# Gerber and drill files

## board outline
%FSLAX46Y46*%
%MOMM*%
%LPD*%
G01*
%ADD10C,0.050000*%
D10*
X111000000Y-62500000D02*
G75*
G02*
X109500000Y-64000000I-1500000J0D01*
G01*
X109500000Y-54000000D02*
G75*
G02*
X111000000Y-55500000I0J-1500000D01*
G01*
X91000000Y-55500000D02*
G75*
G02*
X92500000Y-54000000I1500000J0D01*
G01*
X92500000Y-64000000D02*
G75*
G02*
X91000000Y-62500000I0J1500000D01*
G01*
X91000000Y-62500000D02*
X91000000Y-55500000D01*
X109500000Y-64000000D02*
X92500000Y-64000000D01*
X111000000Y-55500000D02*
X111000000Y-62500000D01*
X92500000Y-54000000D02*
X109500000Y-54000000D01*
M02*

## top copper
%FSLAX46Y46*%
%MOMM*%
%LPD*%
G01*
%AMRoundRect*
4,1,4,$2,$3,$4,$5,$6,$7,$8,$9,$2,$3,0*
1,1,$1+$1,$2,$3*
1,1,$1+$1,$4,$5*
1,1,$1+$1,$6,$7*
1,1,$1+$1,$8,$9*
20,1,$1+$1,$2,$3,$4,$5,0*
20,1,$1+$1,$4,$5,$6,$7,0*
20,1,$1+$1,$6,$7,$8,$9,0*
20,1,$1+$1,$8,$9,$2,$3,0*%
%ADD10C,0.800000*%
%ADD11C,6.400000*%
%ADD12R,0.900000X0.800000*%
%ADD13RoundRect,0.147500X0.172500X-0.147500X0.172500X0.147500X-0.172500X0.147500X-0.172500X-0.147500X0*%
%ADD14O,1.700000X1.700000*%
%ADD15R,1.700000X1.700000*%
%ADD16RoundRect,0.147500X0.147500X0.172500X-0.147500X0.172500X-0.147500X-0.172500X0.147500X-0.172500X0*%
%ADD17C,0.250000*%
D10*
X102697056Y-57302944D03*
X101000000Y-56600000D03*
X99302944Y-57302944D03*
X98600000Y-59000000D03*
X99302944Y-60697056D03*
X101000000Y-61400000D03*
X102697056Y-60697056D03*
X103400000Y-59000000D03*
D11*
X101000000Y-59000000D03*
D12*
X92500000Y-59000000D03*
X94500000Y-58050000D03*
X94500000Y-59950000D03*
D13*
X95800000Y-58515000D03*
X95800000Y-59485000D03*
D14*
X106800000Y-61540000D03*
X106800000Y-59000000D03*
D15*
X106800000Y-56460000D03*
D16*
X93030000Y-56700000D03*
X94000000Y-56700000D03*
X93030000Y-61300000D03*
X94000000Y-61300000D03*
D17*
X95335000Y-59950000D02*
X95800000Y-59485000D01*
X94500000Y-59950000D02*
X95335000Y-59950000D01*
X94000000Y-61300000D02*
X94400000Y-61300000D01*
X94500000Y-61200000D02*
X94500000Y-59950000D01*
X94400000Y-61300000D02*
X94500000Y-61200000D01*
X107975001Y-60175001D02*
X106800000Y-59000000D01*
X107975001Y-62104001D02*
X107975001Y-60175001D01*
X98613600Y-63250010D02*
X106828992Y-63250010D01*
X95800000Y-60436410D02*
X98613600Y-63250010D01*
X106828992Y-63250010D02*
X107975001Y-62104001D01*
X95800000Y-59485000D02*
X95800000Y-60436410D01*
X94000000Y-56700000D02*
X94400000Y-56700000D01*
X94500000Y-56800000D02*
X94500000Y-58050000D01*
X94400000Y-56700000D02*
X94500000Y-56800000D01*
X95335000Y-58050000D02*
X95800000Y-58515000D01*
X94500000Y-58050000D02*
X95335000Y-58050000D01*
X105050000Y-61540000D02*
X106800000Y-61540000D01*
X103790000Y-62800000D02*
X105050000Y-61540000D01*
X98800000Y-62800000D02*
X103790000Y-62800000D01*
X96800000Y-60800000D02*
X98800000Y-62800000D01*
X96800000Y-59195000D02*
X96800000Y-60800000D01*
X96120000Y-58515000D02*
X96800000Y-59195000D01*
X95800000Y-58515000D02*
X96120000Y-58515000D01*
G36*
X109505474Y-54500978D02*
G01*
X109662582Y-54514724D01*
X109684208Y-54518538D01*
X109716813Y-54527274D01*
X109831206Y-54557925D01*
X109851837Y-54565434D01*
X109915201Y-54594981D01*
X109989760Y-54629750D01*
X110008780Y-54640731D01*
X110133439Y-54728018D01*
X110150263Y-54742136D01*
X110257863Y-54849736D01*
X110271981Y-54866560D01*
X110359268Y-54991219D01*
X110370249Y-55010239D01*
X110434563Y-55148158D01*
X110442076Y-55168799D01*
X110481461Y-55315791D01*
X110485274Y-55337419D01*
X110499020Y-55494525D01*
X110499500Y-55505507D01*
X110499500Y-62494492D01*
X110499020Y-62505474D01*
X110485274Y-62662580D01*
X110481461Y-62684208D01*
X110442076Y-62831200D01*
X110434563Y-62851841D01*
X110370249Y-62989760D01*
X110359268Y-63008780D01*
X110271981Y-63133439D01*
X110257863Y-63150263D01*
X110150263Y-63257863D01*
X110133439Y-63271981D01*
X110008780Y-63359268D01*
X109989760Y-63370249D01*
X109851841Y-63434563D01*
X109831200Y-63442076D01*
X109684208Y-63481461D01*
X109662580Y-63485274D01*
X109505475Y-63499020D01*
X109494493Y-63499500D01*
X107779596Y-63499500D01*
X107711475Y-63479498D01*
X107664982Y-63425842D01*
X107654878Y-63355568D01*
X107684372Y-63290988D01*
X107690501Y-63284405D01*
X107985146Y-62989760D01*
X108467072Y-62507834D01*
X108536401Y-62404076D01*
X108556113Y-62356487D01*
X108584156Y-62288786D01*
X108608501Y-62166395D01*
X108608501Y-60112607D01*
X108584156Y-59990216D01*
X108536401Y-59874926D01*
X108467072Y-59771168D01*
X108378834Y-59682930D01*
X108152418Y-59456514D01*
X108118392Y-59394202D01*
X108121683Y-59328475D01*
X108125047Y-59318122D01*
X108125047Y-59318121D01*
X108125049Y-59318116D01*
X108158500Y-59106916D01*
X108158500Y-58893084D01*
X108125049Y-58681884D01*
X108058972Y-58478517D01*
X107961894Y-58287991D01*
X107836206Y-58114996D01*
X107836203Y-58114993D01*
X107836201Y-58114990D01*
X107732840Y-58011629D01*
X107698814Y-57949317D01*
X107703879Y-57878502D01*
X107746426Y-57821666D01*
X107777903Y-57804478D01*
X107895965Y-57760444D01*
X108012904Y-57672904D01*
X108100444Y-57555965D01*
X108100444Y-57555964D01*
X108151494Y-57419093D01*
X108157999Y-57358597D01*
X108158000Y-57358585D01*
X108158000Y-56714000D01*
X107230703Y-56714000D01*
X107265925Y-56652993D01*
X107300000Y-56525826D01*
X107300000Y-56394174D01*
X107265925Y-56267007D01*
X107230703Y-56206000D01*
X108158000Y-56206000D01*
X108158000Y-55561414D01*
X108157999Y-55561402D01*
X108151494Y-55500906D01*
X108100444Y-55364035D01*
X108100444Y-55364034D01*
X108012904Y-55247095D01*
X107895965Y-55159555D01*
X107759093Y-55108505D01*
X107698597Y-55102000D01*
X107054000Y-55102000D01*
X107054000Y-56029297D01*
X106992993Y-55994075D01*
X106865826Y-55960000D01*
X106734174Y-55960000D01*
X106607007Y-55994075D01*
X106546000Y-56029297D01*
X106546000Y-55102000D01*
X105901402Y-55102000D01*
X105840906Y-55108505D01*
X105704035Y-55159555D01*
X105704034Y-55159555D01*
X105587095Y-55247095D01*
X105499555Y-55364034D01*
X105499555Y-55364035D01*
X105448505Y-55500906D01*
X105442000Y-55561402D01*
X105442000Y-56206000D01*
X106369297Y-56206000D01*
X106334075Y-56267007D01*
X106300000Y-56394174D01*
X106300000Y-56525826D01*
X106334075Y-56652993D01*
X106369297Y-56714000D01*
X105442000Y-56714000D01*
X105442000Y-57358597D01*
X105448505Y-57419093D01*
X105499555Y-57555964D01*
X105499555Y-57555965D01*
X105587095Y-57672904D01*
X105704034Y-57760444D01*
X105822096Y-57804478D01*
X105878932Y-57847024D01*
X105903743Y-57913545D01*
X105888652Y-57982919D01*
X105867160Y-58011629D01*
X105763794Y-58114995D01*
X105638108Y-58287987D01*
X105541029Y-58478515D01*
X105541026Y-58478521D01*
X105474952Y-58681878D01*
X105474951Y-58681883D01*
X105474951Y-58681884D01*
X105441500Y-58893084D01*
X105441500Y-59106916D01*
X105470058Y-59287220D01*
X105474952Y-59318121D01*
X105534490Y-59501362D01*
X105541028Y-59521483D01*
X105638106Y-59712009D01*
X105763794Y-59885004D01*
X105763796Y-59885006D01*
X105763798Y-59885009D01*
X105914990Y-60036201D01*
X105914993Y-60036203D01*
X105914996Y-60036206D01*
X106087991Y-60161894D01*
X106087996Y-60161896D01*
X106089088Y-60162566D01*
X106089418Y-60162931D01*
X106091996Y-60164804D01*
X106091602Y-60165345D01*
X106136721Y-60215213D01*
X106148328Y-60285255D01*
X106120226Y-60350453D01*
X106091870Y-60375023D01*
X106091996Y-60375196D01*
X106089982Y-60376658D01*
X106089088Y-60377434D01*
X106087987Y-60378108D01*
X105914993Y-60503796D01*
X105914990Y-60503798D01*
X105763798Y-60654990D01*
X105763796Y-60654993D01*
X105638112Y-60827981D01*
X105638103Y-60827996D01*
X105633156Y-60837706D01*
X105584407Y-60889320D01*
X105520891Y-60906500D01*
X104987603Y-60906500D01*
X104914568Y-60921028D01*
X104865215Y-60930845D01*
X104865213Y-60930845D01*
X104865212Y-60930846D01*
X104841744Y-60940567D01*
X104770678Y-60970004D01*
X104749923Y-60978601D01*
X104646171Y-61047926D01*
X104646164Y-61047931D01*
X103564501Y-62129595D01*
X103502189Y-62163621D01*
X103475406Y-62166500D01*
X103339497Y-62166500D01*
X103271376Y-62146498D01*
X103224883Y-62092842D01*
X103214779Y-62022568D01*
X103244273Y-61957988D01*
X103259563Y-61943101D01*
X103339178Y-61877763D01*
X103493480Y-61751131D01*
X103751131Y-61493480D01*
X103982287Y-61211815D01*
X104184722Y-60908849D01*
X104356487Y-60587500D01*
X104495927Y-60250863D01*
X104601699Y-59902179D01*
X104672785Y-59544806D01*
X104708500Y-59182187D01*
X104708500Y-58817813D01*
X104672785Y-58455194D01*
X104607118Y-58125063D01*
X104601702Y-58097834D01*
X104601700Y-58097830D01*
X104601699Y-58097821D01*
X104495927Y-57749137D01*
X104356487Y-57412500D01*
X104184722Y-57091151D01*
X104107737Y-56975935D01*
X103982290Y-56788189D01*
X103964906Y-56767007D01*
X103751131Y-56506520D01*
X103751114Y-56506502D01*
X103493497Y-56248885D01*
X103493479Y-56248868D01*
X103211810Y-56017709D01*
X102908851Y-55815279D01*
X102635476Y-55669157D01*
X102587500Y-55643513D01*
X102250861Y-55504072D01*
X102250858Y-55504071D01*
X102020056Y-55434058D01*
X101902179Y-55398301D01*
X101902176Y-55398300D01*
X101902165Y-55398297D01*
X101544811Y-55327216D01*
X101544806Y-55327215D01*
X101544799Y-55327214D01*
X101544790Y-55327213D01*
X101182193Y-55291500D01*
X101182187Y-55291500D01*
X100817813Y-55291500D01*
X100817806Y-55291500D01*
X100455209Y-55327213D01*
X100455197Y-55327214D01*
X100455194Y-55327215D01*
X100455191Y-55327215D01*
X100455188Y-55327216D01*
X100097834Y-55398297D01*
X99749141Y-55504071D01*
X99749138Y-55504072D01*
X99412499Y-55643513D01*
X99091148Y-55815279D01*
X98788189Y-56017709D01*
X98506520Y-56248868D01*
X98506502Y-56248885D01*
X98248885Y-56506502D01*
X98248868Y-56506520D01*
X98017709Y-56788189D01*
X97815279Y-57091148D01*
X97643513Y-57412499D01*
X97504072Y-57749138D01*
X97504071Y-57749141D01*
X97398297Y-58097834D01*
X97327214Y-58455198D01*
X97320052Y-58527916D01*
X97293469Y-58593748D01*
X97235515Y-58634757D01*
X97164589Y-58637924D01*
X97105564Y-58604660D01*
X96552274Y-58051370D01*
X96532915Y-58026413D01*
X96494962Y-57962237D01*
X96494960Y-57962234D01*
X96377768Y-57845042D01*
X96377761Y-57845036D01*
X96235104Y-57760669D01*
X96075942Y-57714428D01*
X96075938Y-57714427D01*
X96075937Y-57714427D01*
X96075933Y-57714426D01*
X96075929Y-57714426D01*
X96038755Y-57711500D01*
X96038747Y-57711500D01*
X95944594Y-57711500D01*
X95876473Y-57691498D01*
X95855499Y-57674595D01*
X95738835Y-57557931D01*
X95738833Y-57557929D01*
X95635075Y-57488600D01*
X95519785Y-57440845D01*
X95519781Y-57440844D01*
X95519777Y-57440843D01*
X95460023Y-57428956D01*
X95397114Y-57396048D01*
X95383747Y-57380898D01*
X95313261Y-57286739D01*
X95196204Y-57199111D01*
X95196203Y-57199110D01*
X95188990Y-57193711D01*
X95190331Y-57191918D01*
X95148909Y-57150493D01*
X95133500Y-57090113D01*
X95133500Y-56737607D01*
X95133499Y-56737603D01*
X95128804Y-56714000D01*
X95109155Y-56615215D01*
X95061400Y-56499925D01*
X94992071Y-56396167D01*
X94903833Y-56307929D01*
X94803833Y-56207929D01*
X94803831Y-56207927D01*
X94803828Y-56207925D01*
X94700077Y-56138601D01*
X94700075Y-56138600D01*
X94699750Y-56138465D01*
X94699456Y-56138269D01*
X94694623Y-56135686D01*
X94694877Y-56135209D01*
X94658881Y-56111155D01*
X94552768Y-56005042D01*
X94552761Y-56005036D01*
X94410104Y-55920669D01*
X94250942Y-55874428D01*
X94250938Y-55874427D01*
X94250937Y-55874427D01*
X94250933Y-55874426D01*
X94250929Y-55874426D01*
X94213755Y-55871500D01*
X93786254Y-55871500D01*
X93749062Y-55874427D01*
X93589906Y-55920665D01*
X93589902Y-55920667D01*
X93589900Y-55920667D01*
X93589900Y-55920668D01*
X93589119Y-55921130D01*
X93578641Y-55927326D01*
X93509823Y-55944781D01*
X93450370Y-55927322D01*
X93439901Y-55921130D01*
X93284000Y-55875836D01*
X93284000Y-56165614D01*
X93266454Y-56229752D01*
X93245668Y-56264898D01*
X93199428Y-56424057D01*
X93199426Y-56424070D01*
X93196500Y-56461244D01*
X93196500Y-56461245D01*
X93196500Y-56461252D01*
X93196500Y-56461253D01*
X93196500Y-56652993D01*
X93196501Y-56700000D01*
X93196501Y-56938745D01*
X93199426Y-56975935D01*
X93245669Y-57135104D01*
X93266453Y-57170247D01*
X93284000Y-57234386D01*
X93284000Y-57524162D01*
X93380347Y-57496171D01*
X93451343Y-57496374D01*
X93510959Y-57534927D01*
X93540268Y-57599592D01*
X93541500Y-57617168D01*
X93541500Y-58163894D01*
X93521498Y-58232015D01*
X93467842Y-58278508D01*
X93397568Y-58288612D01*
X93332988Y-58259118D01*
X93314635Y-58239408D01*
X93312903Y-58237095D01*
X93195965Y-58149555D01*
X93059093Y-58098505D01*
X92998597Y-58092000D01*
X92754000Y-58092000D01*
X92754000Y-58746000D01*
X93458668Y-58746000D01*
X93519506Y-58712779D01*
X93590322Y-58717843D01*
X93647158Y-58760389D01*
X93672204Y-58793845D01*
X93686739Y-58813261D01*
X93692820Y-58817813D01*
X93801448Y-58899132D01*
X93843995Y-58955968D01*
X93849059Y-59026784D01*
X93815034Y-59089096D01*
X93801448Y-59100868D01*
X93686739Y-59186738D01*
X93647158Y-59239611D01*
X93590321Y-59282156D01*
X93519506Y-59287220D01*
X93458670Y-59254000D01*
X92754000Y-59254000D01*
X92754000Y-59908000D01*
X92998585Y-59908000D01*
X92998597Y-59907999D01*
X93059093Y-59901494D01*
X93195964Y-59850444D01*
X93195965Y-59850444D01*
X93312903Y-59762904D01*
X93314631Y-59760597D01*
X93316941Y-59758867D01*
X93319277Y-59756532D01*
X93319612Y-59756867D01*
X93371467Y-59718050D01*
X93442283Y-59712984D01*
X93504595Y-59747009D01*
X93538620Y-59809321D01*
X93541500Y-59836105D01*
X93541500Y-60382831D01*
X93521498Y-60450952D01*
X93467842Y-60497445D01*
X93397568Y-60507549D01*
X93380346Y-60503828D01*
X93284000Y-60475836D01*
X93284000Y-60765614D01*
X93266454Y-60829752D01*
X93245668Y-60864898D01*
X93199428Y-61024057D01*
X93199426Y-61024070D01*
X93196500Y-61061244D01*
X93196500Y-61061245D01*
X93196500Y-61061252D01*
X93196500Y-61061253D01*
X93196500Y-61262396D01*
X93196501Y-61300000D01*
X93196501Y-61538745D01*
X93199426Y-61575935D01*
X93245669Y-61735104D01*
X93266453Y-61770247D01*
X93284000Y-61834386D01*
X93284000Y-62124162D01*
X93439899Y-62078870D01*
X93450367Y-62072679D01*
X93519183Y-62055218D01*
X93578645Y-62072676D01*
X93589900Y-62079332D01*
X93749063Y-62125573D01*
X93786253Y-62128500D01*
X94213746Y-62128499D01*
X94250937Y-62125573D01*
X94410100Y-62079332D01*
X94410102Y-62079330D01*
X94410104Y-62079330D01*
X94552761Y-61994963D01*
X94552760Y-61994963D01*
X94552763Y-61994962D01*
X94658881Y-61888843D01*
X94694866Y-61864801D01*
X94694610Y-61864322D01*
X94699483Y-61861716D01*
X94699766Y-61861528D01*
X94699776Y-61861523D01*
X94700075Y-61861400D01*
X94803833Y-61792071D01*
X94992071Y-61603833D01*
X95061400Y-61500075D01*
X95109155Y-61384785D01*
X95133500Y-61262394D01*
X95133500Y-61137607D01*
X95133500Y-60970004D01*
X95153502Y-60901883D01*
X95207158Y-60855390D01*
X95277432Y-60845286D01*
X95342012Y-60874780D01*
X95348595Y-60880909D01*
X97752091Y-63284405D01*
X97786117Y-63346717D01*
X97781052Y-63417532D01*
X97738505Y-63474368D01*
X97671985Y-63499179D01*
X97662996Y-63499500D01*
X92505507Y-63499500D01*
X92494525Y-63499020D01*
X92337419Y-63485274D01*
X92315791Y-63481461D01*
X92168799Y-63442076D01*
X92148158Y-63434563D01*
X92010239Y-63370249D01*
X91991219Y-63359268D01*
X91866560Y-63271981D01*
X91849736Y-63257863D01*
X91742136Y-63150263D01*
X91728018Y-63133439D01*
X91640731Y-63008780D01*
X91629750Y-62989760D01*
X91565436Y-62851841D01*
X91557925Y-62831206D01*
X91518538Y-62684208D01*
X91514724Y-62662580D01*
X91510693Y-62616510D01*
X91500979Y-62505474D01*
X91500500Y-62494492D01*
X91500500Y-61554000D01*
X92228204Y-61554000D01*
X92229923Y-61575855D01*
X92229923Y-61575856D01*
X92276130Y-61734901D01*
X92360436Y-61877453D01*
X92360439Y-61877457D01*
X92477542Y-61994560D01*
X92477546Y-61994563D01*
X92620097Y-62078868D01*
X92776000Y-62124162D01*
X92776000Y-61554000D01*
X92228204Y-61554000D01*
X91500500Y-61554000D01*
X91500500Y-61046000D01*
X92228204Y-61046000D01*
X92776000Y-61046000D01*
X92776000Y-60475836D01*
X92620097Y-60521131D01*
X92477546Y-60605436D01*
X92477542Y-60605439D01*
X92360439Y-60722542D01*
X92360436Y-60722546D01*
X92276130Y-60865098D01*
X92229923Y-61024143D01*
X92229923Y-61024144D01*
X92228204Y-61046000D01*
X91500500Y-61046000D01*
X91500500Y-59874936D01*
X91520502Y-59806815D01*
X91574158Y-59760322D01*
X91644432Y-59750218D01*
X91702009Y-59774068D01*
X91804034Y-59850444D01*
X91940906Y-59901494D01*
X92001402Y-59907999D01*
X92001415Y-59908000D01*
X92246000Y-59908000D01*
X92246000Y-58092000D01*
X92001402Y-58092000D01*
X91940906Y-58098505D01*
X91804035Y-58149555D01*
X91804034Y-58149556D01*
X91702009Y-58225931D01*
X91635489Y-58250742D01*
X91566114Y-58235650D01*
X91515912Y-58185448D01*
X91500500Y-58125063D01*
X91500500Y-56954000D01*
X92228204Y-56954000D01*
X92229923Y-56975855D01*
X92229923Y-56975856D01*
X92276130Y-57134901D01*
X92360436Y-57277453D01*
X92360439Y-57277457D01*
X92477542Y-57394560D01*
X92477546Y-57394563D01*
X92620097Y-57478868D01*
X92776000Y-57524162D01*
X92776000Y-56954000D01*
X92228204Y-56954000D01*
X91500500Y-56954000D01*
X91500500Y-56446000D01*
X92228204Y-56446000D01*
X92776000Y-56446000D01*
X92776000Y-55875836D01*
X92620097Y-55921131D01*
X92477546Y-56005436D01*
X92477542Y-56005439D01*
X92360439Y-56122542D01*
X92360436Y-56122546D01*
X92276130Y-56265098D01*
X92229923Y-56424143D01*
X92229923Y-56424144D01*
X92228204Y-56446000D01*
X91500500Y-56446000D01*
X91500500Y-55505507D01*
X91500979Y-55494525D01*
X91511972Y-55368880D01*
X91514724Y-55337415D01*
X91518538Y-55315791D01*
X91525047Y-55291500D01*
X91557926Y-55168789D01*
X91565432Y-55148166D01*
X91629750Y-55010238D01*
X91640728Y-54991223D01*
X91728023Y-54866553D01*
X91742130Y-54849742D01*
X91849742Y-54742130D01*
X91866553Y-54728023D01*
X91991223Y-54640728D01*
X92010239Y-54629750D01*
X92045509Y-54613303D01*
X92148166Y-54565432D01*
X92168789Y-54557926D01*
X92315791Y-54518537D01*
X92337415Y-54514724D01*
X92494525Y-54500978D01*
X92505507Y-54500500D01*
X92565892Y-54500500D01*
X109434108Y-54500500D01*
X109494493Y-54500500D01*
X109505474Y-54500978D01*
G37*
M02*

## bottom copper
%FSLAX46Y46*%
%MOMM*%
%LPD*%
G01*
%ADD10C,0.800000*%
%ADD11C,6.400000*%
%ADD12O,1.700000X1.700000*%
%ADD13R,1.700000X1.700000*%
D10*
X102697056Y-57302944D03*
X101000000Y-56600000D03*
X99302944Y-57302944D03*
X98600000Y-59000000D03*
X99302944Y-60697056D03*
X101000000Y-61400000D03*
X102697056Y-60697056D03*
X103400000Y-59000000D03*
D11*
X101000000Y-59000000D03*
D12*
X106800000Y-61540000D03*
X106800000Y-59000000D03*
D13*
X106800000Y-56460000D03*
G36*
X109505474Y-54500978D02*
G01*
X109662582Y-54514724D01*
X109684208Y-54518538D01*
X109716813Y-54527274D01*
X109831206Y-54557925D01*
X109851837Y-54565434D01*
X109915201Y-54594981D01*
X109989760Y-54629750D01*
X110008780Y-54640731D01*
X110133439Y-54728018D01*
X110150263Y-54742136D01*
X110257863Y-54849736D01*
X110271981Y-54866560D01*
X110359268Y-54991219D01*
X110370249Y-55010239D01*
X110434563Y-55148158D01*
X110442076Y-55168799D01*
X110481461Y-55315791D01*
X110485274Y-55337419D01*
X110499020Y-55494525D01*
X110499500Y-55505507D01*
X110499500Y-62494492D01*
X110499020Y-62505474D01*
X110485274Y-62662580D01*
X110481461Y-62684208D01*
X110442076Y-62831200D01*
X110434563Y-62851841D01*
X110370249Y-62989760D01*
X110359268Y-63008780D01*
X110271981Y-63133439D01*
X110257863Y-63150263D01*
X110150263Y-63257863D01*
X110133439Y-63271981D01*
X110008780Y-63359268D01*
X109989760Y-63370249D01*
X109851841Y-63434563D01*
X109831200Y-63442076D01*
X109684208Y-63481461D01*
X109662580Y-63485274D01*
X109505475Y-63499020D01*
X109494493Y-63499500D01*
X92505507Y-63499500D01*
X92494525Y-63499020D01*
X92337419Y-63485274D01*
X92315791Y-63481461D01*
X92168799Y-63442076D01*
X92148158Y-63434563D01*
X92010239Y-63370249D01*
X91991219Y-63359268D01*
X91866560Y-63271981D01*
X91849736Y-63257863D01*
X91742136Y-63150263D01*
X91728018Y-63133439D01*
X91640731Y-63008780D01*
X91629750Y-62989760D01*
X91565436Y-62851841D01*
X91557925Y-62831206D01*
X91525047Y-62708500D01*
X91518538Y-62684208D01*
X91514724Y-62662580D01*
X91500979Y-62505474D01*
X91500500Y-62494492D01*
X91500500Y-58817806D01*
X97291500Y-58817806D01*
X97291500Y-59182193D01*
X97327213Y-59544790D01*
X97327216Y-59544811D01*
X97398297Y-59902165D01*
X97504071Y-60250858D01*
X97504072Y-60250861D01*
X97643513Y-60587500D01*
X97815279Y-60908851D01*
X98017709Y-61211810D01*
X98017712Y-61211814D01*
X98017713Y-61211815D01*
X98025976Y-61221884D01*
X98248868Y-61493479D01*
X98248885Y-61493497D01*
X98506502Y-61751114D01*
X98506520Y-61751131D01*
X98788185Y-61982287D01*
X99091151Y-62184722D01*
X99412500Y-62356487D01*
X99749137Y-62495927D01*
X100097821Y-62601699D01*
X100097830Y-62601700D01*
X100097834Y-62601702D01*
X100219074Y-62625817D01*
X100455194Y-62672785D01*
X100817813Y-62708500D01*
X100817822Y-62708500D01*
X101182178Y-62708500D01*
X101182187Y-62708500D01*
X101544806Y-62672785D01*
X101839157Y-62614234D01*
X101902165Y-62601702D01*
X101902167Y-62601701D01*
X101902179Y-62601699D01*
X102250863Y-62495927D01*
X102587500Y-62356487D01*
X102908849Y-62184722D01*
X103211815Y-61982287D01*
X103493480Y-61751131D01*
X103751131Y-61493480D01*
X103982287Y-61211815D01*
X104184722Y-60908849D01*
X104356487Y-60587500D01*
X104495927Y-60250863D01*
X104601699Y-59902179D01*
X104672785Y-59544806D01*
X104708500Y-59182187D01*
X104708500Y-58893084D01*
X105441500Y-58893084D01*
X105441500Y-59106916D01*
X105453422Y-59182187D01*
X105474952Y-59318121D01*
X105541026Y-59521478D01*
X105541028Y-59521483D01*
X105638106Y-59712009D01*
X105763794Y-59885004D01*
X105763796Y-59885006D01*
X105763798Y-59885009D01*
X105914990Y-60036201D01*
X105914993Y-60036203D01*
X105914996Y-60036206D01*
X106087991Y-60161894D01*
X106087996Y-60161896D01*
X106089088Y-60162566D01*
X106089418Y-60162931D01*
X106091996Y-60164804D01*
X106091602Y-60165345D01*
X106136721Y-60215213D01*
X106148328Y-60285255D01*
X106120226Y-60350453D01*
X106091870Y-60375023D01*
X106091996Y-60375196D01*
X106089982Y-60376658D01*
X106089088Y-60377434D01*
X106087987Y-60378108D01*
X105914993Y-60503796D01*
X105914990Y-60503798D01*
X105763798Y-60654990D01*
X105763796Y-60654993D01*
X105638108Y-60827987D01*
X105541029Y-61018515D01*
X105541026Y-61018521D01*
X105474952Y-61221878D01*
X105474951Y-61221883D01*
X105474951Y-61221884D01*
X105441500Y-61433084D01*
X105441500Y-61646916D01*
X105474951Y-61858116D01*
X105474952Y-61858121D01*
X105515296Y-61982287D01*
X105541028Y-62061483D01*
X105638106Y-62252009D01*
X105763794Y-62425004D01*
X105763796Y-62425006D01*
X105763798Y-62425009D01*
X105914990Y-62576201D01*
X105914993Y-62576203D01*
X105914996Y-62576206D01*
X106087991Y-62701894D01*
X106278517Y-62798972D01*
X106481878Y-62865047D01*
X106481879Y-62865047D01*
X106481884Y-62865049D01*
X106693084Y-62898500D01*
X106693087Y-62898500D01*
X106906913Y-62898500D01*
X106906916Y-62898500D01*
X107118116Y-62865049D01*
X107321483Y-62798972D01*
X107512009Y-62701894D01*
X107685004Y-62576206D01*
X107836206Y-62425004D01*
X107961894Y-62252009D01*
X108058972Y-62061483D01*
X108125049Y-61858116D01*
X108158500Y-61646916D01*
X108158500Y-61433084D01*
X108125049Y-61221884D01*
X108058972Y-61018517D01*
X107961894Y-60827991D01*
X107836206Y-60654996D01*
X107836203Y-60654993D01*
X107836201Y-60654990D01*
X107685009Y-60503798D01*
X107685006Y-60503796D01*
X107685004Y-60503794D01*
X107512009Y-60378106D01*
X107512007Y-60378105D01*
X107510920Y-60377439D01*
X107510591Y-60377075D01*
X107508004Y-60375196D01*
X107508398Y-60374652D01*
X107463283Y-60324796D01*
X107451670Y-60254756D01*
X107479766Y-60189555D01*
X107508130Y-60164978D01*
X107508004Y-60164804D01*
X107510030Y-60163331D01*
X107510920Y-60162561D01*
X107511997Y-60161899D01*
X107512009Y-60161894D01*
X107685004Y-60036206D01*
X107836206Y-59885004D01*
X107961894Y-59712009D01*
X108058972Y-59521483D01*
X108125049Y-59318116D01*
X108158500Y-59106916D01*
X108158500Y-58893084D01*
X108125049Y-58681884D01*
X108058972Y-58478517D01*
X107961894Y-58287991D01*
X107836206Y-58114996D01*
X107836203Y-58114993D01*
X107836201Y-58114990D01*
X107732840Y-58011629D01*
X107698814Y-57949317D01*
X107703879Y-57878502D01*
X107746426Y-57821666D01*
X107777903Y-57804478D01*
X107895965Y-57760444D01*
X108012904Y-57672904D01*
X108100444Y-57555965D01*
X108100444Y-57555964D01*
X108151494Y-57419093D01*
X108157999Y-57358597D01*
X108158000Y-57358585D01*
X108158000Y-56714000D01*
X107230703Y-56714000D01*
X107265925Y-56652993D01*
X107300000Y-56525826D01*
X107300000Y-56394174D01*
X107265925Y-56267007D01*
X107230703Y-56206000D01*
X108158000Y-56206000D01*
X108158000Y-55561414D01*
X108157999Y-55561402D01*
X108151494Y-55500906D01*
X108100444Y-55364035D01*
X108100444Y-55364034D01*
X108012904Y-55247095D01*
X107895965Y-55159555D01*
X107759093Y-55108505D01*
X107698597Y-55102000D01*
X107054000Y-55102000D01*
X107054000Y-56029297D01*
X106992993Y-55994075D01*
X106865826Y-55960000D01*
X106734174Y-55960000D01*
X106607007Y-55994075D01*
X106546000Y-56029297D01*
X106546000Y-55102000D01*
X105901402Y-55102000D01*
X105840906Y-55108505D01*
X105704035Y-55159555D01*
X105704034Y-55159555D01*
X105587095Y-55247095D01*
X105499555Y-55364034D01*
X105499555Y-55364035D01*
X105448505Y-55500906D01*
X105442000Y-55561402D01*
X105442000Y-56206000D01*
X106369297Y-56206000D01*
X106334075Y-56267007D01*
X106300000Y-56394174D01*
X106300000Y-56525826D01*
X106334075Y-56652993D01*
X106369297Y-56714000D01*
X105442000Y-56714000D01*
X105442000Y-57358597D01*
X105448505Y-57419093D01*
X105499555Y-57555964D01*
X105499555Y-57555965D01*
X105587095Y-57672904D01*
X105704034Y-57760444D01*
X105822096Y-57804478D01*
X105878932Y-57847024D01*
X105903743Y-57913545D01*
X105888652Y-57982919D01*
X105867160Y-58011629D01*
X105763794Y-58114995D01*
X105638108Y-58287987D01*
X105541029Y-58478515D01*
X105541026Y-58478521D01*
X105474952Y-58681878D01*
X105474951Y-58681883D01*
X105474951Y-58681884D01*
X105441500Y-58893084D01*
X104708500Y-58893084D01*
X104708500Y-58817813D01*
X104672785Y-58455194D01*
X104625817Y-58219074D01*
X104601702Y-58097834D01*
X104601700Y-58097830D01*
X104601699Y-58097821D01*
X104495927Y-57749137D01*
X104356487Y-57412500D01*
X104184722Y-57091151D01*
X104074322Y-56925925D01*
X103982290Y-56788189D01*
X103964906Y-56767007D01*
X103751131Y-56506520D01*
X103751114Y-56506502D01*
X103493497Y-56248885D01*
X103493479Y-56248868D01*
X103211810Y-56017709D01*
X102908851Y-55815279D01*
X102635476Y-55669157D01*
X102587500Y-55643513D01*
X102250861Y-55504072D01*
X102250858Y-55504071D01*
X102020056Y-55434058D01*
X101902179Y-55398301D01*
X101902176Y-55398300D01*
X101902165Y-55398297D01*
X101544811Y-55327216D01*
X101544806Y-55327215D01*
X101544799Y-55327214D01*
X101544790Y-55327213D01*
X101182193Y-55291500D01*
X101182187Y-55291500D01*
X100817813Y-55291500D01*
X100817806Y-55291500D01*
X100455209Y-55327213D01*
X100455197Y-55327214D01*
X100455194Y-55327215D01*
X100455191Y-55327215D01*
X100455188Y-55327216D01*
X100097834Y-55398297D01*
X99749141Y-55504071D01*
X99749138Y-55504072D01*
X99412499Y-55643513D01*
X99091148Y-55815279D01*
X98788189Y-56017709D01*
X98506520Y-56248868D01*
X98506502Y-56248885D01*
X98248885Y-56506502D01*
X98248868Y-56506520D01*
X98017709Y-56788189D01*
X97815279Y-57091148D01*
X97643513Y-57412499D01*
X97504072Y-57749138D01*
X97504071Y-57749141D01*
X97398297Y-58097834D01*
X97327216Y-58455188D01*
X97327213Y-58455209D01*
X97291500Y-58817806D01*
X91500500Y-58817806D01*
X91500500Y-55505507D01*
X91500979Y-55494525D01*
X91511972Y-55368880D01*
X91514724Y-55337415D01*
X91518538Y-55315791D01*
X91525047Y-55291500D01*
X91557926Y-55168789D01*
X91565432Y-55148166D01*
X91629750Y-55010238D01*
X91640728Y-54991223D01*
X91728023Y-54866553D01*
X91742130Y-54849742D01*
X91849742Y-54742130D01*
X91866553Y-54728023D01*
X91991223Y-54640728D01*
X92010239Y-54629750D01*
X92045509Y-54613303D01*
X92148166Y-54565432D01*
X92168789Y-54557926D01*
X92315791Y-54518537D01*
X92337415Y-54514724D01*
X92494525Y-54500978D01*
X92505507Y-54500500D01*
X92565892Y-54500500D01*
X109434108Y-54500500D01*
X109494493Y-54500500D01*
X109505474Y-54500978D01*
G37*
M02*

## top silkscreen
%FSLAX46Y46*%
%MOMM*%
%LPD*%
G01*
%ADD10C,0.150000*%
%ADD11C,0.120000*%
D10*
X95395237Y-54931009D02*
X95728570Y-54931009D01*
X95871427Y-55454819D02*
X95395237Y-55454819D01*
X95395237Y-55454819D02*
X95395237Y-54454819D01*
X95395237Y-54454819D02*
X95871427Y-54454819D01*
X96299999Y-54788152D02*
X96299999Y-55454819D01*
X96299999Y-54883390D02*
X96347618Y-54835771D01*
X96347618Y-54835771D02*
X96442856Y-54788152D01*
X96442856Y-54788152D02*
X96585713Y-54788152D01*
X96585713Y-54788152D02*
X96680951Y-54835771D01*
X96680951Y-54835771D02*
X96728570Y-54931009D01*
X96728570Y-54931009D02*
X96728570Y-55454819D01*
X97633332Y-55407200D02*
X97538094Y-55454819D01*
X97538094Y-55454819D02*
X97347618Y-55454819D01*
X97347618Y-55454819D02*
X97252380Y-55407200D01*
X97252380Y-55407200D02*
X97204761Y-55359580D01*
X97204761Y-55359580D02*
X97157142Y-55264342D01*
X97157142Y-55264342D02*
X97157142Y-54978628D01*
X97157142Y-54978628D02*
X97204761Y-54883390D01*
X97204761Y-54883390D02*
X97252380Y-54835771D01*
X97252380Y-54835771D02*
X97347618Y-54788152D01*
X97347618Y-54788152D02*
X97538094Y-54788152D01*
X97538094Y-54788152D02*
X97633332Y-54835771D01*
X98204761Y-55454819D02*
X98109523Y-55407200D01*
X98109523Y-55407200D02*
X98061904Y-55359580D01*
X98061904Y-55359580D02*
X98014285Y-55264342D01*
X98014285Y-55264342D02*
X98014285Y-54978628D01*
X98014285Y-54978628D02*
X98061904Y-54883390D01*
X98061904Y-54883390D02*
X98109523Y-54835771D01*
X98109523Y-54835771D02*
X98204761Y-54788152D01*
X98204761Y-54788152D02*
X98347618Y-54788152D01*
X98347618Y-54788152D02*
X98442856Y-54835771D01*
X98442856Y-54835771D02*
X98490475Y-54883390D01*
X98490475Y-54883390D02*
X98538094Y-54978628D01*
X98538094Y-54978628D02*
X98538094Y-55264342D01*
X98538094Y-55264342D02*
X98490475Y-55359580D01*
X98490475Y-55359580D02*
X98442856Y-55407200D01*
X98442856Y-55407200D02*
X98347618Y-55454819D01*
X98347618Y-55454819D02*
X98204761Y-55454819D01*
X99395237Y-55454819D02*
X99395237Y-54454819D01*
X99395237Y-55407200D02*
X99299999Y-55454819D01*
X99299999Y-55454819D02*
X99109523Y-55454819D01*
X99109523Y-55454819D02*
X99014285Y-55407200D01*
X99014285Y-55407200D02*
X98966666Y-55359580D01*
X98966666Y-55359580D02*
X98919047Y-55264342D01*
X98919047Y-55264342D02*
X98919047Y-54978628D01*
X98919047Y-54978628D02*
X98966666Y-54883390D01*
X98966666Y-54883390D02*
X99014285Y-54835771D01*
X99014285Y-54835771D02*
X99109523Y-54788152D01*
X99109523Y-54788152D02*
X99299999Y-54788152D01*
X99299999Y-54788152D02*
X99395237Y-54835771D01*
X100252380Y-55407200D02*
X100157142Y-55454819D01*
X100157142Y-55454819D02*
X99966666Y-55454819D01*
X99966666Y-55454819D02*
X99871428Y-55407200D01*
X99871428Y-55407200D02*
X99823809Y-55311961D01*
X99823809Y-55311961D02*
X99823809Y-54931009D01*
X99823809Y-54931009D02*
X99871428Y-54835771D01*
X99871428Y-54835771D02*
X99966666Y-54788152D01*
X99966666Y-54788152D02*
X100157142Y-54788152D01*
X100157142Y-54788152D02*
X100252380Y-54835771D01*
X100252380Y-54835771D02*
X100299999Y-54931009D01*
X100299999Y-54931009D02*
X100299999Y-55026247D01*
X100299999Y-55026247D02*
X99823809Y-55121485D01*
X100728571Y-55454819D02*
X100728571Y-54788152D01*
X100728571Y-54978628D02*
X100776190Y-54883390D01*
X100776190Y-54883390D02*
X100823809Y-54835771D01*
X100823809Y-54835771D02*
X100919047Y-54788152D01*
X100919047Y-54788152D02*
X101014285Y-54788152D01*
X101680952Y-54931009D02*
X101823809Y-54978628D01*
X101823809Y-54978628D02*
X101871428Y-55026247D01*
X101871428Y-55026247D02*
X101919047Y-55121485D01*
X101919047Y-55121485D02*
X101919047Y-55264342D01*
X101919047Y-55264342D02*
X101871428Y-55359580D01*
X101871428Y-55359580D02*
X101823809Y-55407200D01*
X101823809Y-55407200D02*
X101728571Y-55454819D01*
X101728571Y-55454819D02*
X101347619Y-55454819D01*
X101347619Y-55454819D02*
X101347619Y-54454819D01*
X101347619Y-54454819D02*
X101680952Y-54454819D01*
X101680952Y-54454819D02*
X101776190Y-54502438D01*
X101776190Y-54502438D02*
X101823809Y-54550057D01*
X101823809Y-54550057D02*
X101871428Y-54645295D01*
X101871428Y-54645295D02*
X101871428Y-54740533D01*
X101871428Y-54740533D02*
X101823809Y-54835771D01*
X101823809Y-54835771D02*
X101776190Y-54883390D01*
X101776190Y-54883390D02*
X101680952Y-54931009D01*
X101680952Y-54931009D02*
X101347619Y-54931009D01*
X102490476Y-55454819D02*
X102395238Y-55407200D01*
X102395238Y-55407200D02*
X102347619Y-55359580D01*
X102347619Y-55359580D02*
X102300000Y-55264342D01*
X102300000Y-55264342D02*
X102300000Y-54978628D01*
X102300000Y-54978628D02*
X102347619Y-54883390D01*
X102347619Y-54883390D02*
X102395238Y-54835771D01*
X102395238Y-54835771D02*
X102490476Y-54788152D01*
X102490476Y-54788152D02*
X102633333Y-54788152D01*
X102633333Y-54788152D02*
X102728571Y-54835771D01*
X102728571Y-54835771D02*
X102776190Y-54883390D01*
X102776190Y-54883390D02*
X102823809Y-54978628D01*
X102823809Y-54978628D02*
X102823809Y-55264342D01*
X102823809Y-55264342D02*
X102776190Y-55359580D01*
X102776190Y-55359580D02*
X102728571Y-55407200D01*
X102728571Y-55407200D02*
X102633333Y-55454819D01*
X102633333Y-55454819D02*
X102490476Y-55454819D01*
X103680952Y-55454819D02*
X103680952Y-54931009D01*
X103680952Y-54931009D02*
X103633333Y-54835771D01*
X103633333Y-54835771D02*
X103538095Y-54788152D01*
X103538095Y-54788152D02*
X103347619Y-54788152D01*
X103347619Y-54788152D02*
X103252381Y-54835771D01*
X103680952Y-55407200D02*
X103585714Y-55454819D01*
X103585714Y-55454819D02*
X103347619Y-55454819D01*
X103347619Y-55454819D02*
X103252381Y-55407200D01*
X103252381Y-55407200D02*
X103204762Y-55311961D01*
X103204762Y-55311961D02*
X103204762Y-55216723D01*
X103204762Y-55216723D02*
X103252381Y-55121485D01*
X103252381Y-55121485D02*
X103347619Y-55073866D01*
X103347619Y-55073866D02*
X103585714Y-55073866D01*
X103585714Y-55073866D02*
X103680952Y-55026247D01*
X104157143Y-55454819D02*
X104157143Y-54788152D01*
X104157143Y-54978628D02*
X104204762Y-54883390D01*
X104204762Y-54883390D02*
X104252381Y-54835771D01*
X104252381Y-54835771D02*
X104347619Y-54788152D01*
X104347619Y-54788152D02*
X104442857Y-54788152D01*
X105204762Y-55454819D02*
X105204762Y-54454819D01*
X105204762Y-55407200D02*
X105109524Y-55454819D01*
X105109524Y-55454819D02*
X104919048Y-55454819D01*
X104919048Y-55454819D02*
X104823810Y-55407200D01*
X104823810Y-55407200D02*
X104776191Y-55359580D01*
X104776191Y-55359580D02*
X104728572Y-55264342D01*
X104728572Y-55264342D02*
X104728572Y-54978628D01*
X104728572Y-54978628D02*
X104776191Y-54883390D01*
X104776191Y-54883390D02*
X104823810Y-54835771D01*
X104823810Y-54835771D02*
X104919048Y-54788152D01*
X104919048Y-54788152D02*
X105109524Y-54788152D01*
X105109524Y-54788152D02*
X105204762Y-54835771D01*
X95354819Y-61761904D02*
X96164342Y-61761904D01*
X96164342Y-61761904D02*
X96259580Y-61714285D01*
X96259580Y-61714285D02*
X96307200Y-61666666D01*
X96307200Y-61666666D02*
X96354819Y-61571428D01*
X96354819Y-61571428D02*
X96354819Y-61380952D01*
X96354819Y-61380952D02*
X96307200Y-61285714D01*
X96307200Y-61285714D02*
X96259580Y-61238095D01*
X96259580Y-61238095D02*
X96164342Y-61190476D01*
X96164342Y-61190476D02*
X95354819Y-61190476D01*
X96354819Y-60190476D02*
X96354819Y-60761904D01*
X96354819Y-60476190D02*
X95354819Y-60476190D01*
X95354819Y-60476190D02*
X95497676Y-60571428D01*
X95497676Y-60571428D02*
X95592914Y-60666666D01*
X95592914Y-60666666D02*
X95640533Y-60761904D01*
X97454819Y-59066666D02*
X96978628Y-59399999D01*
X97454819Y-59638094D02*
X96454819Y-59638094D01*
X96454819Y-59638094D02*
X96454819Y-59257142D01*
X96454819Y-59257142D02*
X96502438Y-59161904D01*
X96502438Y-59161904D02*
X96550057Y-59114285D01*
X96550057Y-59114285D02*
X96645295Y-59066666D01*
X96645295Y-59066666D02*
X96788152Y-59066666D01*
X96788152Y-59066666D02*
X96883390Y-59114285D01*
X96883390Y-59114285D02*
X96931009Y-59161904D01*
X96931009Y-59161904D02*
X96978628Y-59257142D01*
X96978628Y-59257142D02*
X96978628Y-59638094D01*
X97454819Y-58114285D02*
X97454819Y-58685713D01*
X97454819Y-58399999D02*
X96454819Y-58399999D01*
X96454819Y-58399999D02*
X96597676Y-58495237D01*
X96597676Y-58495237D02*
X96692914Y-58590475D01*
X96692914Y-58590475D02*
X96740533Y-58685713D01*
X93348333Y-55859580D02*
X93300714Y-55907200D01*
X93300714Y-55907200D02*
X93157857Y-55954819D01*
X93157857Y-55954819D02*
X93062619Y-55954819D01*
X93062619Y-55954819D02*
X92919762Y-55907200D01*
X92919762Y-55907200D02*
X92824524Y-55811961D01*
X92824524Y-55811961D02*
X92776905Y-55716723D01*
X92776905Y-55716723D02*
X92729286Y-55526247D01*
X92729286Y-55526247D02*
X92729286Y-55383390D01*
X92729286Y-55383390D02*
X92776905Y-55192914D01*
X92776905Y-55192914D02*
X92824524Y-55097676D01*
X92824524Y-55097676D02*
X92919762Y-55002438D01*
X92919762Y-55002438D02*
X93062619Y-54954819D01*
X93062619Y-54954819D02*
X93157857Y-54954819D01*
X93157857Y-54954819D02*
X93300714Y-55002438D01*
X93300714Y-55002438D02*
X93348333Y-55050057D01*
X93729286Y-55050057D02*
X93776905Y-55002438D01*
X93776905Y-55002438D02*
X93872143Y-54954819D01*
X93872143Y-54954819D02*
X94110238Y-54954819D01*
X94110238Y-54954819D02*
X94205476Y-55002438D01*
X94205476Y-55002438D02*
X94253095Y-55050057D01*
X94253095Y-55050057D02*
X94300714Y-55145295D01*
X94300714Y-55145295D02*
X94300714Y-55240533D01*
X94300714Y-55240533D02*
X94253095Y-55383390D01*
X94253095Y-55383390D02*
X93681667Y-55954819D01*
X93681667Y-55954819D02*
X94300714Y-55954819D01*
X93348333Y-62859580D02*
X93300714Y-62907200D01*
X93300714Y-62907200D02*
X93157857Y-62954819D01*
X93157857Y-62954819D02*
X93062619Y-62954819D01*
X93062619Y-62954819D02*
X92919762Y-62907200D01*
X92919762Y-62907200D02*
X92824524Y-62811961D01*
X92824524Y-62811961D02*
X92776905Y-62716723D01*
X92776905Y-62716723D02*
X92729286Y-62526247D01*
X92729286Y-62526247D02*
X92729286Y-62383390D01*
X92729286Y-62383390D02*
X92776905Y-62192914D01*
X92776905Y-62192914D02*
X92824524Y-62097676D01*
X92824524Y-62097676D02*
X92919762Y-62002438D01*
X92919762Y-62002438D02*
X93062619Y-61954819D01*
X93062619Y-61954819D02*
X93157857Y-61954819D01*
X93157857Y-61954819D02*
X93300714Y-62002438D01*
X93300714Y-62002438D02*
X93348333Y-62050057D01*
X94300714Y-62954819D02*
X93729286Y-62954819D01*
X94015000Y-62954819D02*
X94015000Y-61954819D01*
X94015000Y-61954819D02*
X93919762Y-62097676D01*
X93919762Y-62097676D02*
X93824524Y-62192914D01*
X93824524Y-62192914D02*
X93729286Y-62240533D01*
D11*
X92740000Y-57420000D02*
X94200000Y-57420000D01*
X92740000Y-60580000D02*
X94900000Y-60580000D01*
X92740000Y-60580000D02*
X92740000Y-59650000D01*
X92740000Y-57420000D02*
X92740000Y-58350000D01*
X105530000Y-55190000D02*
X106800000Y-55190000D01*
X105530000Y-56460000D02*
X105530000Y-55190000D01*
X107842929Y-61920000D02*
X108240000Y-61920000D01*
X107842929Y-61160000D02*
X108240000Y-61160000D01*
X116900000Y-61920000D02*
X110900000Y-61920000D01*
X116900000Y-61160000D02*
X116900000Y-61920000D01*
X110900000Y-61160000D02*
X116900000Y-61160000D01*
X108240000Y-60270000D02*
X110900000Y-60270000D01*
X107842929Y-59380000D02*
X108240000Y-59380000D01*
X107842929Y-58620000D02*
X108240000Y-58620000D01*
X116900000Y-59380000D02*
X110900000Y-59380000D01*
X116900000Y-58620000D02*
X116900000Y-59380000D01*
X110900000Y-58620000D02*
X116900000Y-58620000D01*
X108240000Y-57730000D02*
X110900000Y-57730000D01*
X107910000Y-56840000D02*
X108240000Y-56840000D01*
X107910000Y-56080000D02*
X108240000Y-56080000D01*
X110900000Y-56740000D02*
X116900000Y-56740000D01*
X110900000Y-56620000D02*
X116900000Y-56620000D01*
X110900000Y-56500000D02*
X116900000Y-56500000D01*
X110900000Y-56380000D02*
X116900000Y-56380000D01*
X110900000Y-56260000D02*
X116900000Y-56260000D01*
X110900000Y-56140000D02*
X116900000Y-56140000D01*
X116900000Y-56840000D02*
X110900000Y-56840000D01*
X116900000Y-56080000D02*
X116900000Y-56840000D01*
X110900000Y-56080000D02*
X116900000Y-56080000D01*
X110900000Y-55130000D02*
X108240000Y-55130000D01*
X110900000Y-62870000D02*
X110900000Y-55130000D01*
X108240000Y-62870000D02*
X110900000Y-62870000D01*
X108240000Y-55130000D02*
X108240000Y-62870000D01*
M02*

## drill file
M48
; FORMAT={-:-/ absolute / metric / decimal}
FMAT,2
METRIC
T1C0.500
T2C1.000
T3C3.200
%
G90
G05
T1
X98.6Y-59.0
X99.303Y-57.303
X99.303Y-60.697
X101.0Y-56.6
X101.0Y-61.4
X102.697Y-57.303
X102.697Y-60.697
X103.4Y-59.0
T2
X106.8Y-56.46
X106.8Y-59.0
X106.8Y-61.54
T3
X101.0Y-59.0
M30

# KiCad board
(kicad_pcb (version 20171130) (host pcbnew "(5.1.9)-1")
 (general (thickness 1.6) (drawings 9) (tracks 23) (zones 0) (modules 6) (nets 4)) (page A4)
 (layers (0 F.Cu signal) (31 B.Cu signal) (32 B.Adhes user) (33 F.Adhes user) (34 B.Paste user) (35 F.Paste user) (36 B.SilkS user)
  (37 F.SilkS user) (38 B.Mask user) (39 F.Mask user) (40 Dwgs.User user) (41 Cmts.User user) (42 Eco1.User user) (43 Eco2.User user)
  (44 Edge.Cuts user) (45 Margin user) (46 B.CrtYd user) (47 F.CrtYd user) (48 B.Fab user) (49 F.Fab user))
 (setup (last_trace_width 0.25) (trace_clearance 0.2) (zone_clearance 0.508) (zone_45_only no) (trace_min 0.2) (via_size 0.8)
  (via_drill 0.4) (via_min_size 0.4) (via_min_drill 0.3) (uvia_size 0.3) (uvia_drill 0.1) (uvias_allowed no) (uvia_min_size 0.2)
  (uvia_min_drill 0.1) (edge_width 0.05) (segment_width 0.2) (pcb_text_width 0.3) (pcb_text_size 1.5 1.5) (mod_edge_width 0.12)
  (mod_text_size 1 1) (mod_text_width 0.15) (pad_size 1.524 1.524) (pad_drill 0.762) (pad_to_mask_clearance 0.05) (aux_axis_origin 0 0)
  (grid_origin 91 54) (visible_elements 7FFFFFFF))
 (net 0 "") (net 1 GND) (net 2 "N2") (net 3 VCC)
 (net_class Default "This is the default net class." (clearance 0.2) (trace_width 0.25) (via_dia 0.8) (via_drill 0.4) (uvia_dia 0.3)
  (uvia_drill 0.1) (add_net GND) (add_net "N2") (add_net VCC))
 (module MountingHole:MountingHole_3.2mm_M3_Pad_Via (layer F.Cu) (at 101 59)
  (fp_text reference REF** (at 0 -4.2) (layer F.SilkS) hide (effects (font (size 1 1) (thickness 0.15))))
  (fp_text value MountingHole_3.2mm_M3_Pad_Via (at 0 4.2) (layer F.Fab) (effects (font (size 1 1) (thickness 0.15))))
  (pad 1 thru_hole circle (at 1.697056 -1.697056) (size 0.8 0.8) (drill 0.5) (layers *.Cu *.Mask))
  (pad 1 thru_hole circle (at 0 -2.4) (size 0.8 0.8) (drill 0.5) (layers *.Cu *.Mask))
  (pad 1 thru_hole circle (at -1.697056 -1.697056) (size 0.8 0.8) (drill 0.5) (layers *.Cu *.Mask))
  (pad 1 thru_hole circle (at -2.4 0) (size 0.8 0.8) (drill 0.5) (layers *.Cu *.Mask))
  (pad 1 thru_hole circle (at -1.697056 1.697056) (size 0.8 0.8) (drill 0.5) (layers *.Cu *.Mask))
  (pad 1 thru_hole circle (at 0 2.4) (size 0.8 0.8) (drill 0.5) (layers *.Cu *.Mask))
  (pad 1 thru_hole circle (at 1.697056 1.697056) (size 0.8 0.8) (drill 0.5) (layers *.Cu *.Mask))
  (pad 1 thru_hole circle (at 2.4 0) (size 0.8 0.8) (drill 0.5) (layers *.Cu *.Mask))
  (pad 1 thru_hole circle (at 0 0) (size 6.4 6.4) (drill 3.2) (layers *.Cu *.Mask)))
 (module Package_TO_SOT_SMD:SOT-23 (layer F.Cu) (at 93.5 59 180)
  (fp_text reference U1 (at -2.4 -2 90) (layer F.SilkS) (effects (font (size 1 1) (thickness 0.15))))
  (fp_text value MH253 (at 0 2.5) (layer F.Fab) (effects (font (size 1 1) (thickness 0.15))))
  (fp_line (start 0.76 1.58) (end -0.7 1.58) (layer F.SilkS) (width 0.12))
  (fp_line (start 0.76 -1.58) (end -1.4 -1.58) (layer F.SilkS) (width 0.12))
  (fp_line (start 0.76 -1.58) (end 0.76 -0.65) (layer F.SilkS) (width 0.12))
  (fp_line (start 0.76 1.58) (end 0.76 0.65) (layer F.SilkS) (width 0.12))
  (pad 3 smd rect (at 1 0 180) (size 0.9 0.8) (layers F.Cu F.Paste F.Mask) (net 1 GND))
  (pad 2 smd rect (at -1 0.95 180) (size 0.9 0.8) (layers F.Cu F.Paste F.Mask) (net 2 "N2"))
  (pad 1 smd rect (at -1 -0.95 180) (size 0.9 0.8) (layers F.Cu F.Paste F.Mask) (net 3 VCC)))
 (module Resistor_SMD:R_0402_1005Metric (layer F.Cu) (at 95.8 59 90)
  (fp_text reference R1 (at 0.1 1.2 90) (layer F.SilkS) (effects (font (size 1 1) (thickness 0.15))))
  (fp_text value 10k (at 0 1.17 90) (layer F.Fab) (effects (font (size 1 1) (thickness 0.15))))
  (pad 2 smd roundrect (at 0.485 0 90) (size 0.59 0.64) (layers F.Cu F.Paste F.Mask) (roundrect_rratio 0.25) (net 2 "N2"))
  (pad 1 smd roundrect (at -0.485 0 90) (size 0.59 0.64) (layers F.Cu F.Paste F.Mask) (roundrect_rratio 0.25) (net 3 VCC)))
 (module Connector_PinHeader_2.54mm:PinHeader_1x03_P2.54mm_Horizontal (layer F.Cu) (at 106.8 56.46)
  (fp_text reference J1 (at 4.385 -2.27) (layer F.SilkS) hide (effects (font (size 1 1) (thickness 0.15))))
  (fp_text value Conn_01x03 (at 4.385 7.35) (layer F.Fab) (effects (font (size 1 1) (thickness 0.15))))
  (fp_line (start -1.27 -1.27) (end 0 -1.27) (layer F.SilkS) (width 0.12))
  (fp_line (start -1.27 0) (end -1.27 -1.27) (layer F.SilkS) (width 0.12))
  (fp_line (start 1.042929 5.46) (end 1.44 5.46) (layer F.SilkS) (width 0.12))
  (fp_line (start 1.042929 4.7) (end 1.44 4.7) (layer F.SilkS) (width 0.12))
  (fp_line (start 10.1 5.46) (end 4.1 5.46) (layer F.SilkS) (width 0.12))
  (fp_line (start 10.1 4.7) (end 10.1 5.46) (layer F.SilkS) (width 0.12))
  (fp_line (start 4.1 4.7) (end 10.1 4.7) (layer F.SilkS) (width 0.12))
  (fp_line (start 1.44 3.81) (end 4.1 3.81) (layer F.SilkS) (width 0.12))
  (fp_line (start 1.042929 2.92) (end 1.44 2.92) (layer F.SilkS) (width 0.12))
  (fp_line (start 1.042929 2.16) (end 1.44 2.16) (layer F.SilkS) (width 0.12))
  (fp_line (start 10.1 2.92) (end 4.1 2.92) (layer F.SilkS) (width 0.12))
  (fp_line (start 10.1 2.16) (end 10.1 2.92) (layer F.SilkS) (width 0.12))
  (fp_line (start 4.1 2.16) (end 10.1 2.16) (layer F.SilkS) (width 0.12))
  (fp_line (start 1.44 1.27) (end 4.1 1.27) (layer F.SilkS) (width 0.12))
  (fp_line (start 1.11 0.38) (end 1.44 0.38) (layer F.SilkS) (width 0.12))
  (fp_line (start 1.11 -0.38) (end 1.44 -0.38) (layer F.SilkS) (width 0.12))
  (fp_line (start 4.1 0.28) (end 10.1 0.28) (layer F.SilkS) (width 0.12))
  (fp_line (start 4.1 0.16) (end 10.1 0.16) (layer F.SilkS) (width 0.12))
  (fp_line (start 4.1 0.04) (end 10.1 0.04) (layer F.SilkS) (width 0.12))
  (fp_line (start 4.1 -0.08) (end 10.1 -0.08) (layer F.SilkS) (width 0.12))
  (fp_line (start 4.1 -0.2) (end 10.1 -0.2) (layer F.SilkS) (width 0.12))
  (fp_line (start 4.1 -0.32) (end 10.1 -0.32) (layer F.SilkS) (width 0.12))
  (fp_line (start 10.1 0.38) (end 4.1 0.38) (layer F.SilkS) (width 0.12))
  (fp_line (start 10.1 -0.38) (end 10.1 0.38) (layer F.SilkS) (width 0.12))
  (fp_line (start 4.1 -0.38) (end 10.1 -0.38) (layer F.SilkS) (width 0.12))
  (fp_line (start 4.1 -1.33) (end 1.44 -1.33) (layer F.SilkS) (width 0.12))
  (fp_line (start 4.1 6.41) (end 4.1 -1.33) (layer F.SilkS) (width 0.12))
  (fp_line (start 1.44 6.41) (end 4.1 6.41) (layer F.SilkS) (width 0.12))
  (fp_line (start 1.44 -1.33) (end 1.44 6.41) (layer F.SilkS) (width 0.12))
  (pad 3 thru_hole oval (at 0 5.08) (size 1.7 1.7) (drill 1) (layers *.Cu *.Mask) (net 2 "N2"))
  (pad 2 thru_hole oval (at 0 2.54) (size 1.7 1.7) (drill 1) (layers *.Cu *.Mask) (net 3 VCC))
  (pad 1 thru_hole rect (at 0 0) (size 1.7 1.7) (drill 1) (layers *.Cu *.Mask) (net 1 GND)))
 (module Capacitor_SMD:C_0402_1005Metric (layer F.Cu) (at 93.515 56.7 180)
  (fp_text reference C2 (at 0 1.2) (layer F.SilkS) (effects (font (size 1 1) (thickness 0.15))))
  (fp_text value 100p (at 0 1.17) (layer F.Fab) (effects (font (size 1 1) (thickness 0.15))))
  (pad 2 smd roundrect (at 0.485 0 180) (size 0.59 0.64) (layers F.Cu F.Paste F.Mask) (roundrect_rratio 0.25) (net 1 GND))
  (pad 1 smd roundrect (at -0.485 0 180) (size 0.59 0.64) (layers F.Cu F.Paste F.Mask) (roundrect_rratio 0.25) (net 2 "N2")))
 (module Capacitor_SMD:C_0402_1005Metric (layer F.Cu) (at 93.515 61.3 180)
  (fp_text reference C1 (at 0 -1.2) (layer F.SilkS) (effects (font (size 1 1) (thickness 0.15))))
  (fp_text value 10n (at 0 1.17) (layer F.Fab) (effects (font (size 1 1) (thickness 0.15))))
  (pad 2 smd roundrect (at 0.485 0 180) (size 0.59 0.64) (layers F.Cu F.Paste F.Mask) (roundrect_rratio 0.25) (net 1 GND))
  (pad 1 smd roundrect (at -0.485 0 180) (size 0.59 0.64) (layers F.Cu F.Paste F.Mask) (roundrect_rratio 0.25) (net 3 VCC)))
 (gr_arc (start 109.5 62.5) (end 109.5 64) (angle -90) (layer Edge.Cuts) (width 0.05))
 (gr_arc (start 109.5 55.5) (end 111 55.5) (angle -90) (layer Edge.Cuts) (width 0.05))
 (gr_arc (start 92.5 55.5) (end 92.5 54) (angle -90) (layer Edge.Cuts) (width 0.05))
 (gr_arc (start 92.5 62.5) (end 91 62.5) (angle -90) (layer Edge.Cuts) (width 0.05))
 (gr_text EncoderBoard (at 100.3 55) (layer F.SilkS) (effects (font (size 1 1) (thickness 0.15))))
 (gr_line (start 91 62.5) (end 91 55.5) (layer Edge.Cuts) (width 0.05))
 (gr_line (start 109.5 64) (end 92.5 64) (layer Edge.Cuts) (width 0.05))
 (gr_line (start 111 55.5) (end 111 62.5) (layer Edge.Cuts) (width 0.05))
 (gr_line (start 92.5 54) (end 109.5 54) (layer Edge.Cuts) (width 0.05))
 (segment (start 95.335 59.95) (end 95.8 59.485) (width 0.25) (layer F.Cu) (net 3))
 (segment (start 94.5 59.95) (end 95.335 59.95) (width 0.25) (layer F.Cu) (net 3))
 (segment (start 94 61.3) (end 94.4 61.3) (width 0.25) (layer F.Cu) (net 3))
 (segment (start 94.5 61.2) (end 94.5 59.95) (width 0.25) (layer F.Cu) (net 3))
 (segment (start 94.4 61.3) (end 94.5 61.2) (width 0.25) (layer F.Cu) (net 3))
 (segment (start 107.975001 60.175001) (end 106.8 59) (width 0.25) (layer F.Cu) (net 3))
 (segment (start 107.975001 62.104001) (end 107.975001 60.175001) (width 0.25) (layer F.Cu) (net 3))
 (segment (start 98.6136 63.25001) (end 106.828992 63.25001) (width 0.25) (layer F.Cu) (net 3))
 (segment (start 95.8 60.43641) (end 98.6136 63.25001) (width 0.25) (layer F.Cu) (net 3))
 (segment (start 106.828992 63.25001) (end 107.975001 62.104001) (width 0.25) (layer F.Cu) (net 3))
 (segment (start 95.8 59.485) (end 95.8 60.43641) (width 0.25) (layer F.Cu) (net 3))
 (segment (start 94 56.7) (end 94.4 56.7) (width 0.25) (layer F.Cu) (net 2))
 (segment (start 94.5 56.8) (end 94.5 58.05) (width 0.25) (layer F.Cu) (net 2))
 (segment (start 94.4 56.7) (end 94.5 56.8) (width 0.25) (layer F.Cu) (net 2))
 (segment (start 95.335 58.05) (end 95.8 58.515) (width 0.25) (layer F.Cu) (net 2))
 (segment (start 94.5 58.05) (end 95.335 58.05) (width 0.25) (layer F.Cu) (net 2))
 (segment (start 105.05 61.54) (end 106.8 61.54) (width 0.25) (layer F.Cu) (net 2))
 (segment (start 103.79 62.8) (end 105.05 61.54) (width 0.25) (layer F.Cu) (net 2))
 (segment (start 98.8 62.8) (end 103.79 62.8) (width 0.25) (layer F.Cu) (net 2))
 (segment (start 96.8 60.8) (end 98.8 62.8) (width 0.25) (layer F.Cu) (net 2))
 (segment (start 96.8 59.195) (end 96.8 60.8) (width 0.25) (layer F.Cu) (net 2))
 (segment (start 96.12 58.515) (end 96.8 59.195) (width 0.25) (layer F.Cu) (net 2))
 (segment (start 95.8 58.515) (end 96.12 58.515) (width 0.25) (layer F.Cu) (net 2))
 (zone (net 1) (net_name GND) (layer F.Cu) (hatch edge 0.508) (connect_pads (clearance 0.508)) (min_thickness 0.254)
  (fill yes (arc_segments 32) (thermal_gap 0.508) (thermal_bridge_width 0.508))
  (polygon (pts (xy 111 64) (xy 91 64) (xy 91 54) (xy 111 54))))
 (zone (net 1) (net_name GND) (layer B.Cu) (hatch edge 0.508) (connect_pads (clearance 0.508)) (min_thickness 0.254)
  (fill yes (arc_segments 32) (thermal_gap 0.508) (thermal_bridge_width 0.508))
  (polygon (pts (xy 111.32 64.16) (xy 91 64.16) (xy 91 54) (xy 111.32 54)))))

